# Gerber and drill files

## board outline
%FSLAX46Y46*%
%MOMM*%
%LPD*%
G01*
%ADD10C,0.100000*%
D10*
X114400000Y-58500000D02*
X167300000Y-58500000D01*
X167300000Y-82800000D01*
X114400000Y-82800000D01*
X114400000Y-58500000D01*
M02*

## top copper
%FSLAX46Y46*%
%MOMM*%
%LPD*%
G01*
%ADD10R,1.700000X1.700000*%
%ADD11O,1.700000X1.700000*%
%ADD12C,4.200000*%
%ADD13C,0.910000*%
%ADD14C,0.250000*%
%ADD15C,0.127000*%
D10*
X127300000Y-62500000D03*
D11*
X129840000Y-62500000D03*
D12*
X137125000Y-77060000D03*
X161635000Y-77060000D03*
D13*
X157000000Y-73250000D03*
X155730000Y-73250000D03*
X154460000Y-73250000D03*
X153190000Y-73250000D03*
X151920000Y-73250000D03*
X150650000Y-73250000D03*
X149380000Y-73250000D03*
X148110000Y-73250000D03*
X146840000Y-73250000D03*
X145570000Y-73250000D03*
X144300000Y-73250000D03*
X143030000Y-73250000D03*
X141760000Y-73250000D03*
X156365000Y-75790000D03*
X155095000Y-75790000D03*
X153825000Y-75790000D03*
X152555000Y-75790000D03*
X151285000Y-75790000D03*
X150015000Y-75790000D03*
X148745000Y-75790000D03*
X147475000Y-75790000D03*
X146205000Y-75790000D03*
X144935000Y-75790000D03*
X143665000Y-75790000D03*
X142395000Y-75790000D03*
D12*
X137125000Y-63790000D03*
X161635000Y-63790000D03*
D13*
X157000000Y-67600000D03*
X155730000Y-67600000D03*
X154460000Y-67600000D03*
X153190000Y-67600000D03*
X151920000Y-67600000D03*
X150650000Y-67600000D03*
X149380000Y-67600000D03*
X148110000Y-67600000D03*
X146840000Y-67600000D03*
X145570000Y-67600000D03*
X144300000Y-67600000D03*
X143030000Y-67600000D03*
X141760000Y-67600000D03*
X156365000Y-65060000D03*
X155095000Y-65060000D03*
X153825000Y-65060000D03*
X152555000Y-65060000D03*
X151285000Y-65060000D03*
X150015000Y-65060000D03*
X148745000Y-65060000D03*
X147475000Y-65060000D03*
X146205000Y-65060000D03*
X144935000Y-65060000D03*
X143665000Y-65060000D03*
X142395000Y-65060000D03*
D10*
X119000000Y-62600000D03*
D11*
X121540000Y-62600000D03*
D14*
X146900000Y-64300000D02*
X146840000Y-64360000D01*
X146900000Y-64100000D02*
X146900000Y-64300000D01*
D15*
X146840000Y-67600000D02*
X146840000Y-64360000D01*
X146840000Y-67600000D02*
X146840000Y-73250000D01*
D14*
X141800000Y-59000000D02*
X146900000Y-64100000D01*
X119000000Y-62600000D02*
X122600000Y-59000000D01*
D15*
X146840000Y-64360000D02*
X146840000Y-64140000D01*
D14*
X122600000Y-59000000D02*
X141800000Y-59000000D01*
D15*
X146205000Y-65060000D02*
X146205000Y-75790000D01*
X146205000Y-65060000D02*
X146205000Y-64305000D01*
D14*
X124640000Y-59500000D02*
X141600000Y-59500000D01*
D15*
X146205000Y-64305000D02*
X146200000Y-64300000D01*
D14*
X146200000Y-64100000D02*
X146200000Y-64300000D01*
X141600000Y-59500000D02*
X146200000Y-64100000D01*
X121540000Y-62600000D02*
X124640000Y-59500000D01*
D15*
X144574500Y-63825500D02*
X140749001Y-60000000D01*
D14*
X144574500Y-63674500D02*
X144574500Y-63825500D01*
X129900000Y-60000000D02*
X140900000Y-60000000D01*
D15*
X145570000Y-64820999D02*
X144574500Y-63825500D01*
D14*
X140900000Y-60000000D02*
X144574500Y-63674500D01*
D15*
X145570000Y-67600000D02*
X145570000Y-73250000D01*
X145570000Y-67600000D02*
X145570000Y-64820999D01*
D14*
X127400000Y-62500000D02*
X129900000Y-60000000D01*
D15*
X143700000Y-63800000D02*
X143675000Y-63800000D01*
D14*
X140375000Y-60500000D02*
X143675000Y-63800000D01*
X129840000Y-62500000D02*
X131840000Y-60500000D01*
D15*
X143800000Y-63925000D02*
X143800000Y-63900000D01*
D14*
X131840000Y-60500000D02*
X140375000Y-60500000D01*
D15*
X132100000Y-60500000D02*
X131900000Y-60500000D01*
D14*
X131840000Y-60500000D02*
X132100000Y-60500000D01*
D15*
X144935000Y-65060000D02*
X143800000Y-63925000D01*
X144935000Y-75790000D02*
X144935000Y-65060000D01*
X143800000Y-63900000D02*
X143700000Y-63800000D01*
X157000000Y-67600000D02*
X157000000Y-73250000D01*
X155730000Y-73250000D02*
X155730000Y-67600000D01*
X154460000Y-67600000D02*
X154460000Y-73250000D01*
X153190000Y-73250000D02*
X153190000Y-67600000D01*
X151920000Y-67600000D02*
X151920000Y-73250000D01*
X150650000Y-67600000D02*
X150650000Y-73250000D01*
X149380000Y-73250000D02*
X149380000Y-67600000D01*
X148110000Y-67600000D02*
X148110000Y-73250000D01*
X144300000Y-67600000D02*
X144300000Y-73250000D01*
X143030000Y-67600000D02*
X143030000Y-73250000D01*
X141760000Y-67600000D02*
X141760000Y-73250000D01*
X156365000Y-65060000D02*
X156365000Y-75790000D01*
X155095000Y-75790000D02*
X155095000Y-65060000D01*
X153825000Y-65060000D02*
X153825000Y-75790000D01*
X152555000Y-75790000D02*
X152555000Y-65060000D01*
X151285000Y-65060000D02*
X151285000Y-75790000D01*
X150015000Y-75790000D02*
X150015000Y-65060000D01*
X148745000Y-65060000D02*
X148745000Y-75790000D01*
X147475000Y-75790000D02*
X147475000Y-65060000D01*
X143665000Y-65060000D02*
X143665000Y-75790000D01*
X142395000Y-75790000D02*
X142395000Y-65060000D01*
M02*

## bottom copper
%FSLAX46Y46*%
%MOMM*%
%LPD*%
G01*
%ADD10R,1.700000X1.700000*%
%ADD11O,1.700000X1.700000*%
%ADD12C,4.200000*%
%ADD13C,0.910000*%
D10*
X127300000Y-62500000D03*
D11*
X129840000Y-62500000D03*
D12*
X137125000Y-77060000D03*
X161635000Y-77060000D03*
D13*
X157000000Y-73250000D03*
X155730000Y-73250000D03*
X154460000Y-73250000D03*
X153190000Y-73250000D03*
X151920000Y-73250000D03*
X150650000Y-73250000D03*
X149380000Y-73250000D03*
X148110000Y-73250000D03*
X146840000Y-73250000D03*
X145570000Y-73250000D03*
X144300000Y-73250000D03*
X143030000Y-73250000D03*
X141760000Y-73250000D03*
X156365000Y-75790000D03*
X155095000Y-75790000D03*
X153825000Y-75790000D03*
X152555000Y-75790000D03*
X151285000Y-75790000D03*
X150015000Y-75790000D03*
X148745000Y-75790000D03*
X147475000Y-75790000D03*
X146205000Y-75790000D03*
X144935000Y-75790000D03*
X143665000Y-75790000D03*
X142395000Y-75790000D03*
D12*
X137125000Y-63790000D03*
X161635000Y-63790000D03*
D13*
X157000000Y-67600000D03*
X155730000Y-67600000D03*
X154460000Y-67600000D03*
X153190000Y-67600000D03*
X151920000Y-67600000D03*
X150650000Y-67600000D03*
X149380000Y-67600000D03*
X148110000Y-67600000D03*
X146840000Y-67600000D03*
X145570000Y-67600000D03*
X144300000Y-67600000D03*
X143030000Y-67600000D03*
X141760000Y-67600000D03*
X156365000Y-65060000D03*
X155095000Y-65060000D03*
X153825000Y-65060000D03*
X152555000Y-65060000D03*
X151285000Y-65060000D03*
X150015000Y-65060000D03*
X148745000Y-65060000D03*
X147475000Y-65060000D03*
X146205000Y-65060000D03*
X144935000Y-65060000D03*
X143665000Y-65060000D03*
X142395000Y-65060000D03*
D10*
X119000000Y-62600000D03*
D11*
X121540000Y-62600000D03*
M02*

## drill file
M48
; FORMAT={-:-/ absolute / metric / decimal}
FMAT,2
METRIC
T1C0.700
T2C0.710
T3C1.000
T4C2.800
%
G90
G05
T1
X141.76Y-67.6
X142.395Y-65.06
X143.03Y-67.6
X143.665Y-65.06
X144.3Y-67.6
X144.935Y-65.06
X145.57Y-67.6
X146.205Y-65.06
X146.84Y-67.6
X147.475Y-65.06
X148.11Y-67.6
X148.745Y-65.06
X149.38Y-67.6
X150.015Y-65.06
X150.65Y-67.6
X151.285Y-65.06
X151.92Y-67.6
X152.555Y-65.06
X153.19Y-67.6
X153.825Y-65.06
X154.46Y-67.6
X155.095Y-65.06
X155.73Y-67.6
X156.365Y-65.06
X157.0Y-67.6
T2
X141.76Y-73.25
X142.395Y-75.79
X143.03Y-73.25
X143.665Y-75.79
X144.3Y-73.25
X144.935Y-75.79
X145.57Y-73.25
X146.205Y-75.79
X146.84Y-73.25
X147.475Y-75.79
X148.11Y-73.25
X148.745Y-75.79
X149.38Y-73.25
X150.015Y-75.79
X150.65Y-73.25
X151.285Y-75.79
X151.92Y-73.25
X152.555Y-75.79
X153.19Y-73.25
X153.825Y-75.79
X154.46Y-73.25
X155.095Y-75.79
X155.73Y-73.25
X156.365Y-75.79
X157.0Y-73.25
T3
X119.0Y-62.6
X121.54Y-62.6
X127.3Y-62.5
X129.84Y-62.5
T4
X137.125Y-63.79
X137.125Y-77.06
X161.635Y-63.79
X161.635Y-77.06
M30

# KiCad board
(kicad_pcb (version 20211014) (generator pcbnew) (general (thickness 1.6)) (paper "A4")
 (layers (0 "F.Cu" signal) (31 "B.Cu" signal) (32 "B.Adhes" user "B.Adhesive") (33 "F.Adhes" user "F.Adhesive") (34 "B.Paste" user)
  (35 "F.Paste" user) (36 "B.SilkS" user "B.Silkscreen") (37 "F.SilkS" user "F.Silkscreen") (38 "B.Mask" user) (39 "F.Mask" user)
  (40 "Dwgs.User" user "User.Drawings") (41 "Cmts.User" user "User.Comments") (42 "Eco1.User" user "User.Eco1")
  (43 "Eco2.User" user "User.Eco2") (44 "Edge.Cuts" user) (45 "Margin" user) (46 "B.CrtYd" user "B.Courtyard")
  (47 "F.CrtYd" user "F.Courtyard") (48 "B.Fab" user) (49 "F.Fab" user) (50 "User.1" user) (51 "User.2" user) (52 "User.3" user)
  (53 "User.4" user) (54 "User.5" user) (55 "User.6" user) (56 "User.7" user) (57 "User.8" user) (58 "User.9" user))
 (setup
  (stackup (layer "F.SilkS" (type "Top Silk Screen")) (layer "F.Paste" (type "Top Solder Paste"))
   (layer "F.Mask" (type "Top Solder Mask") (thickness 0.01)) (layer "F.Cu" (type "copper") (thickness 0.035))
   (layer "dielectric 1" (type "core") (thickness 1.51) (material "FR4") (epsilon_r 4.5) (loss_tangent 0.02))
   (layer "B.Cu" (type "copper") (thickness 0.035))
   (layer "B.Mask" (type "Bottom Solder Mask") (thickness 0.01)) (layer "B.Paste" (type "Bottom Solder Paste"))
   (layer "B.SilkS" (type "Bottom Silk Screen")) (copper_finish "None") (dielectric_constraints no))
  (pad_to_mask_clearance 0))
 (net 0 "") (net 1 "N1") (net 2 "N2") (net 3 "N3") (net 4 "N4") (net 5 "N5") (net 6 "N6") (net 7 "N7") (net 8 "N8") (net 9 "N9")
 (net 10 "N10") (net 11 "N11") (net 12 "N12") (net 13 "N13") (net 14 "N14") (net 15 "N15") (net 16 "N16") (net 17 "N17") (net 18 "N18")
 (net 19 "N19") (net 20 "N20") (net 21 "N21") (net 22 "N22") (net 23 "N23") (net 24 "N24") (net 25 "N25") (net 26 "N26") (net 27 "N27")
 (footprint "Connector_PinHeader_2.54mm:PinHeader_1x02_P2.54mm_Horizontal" (layer "F.Cu") (at 127.3 62.5 90)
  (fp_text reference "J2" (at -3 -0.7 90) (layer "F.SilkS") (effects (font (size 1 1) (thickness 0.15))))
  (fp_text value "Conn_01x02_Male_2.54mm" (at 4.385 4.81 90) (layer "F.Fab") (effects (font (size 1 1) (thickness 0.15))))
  (pad "1" thru_hole rect (at 0 0 90) (size 1.7 1.7) (drill 1) (layers *.Cu *.Mask) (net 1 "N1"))
  (pad "2" thru_hole oval (at 0 2.54 90) (size 1.7 1.7) (drill 1) (layers *.Cu *.Mask) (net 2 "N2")))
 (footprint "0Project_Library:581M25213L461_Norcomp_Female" (layer "F.Cu") (at 157 73.25)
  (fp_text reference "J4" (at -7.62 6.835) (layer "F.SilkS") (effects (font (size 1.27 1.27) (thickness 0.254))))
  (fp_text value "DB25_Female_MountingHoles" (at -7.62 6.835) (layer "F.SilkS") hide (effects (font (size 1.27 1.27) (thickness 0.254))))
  (pad "0" thru_hole circle (at -19.875 3.81) (size 4.2 4.2) (drill 2.8) (layers *.Cu *.Mask) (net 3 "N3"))
  (pad "0" thru_hole circle (at 4.635 3.81) (size 4.2 4.2) (drill 2.8) (layers *.Cu *.Mask) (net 3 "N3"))
  (pad "1" thru_hole circle (at 0 0) (size 0.91 0.91) (drill 0.71) (layers *.Cu *.Mask) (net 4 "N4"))
  (pad "2" thru_hole circle (at -1.27 0) (size 0.91 0.91) (drill 0.71) (layers *.Cu *.Mask) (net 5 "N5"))
  (pad "3" thru_hole circle (at -2.54 0) (size 0.91 0.91) (drill 0.71) (layers *.Cu *.Mask) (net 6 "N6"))
  (pad "4" thru_hole circle (at -3.81 0) (size 0.91 0.91) (drill 0.71) (layers *.Cu *.Mask) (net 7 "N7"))
  (pad "5" thru_hole circle (at -5.08 0) (size 0.91 0.91) (drill 0.71) (layers *.Cu *.Mask) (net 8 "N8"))
  (pad "6" thru_hole circle (at -6.35 0) (size 0.91 0.91) (drill 0.71) (layers *.Cu *.Mask) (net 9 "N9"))
  (pad "7" thru_hole circle (at -7.62 0) (size 0.91 0.91) (drill 0.71) (layers *.Cu *.Mask) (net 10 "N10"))
  (pad "8" thru_hole circle (at -8.89 0) (size 0.91 0.91) (drill 0.71) (layers *.Cu *.Mask) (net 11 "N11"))
  (pad "9" thru_hole circle (at -10.16 0) (size 0.91 0.91) (drill 0.71) (layers *.Cu *.Mask) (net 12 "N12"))
  (pad "10" thru_hole circle (at -11.43 0) (size 0.91 0.91) (drill 0.71) (layers *.Cu *.Mask) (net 1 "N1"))
  (pad "11" thru_hole circle (at -12.7 0) (size 0.91 0.91) (drill 0.71) (layers *.Cu *.Mask) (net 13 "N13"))
  (pad "12" thru_hole circle (at -13.97 0) (size 0.91 0.91) (drill 0.71) (layers *.Cu *.Mask) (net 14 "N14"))
  (pad "13" thru_hole circle (at -15.24 0) (size 0.91 0.91) (drill 0.71) (layers *.Cu *.Mask) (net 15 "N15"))
  (pad "14" thru_hole circle (at -0.635 2.54) (size 0.91 0.91) (drill 0.71) (layers *.Cu *.Mask) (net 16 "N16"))
  (pad "15" thru_hole circle (at -1.905 2.54) (size 0.91 0.91) (drill 0.71) (layers *.Cu *.Mask) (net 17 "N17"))
  (pad "16" thru_hole circle (at -3.175 2.54) (size 0.91 0.91) (drill 0.71) (layers *.Cu *.Mask) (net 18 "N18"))
  (pad "17" thru_hole circle (at -4.445 2.54) (size 0.91 0.91) (drill 0.71) (layers *.Cu *.Mask) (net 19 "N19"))
  (pad "18" thru_hole circle (at -5.715 2.54) (size 0.91 0.91) (drill 0.71) (layers *.Cu *.Mask) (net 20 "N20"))
  (pad "19" thru_hole circle (at -6.985 2.54) (size 0.91 0.91) (drill 0.71) (layers *.Cu *.Mask) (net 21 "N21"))
  (pad "20" thru_hole circle (at -8.255 2.54) (size 0.91 0.91) (drill 0.71) (layers *.Cu *.Mask) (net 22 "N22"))
  (pad "21" thru_hole circle (at -9.525 2.54) (size 0.91 0.91) (drill 0.71) (layers *.Cu *.Mask) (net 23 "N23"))
  (pad "22" thru_hole circle (at -10.795 2.54) (size 0.91 0.91) (drill 0.71) (layers *.Cu *.Mask) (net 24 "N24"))
  (pad "23" thru_hole circle (at -12.065 2.54) (size 0.91 0.91) (drill 0.71) (layers *.Cu *.Mask) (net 2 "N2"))
  (pad "24" thru_hole circle (at -13.335 2.54) (size 0.91 0.91) (drill 0.71) (layers *.Cu *.Mask) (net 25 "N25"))
  (pad "25" thru_hole circle (at -14.605 2.54) (size 0.91 0.91) (drill 0.71) (layers *.Cu *.Mask) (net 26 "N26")))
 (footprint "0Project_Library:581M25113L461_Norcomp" (layer "F.Cu") (at 157 67.6 180)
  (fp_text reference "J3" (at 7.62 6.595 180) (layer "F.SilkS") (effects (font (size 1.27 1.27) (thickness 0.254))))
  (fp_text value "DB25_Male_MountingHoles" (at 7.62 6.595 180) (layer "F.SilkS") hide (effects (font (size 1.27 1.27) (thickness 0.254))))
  (pad "0" thru_hole circle (at 19.875 3.81 180) (size 4.2 4.2) (drill 2.8) (layers *.Cu *.Mask) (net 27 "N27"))
  (pad "0" thru_hole circle (at -4.635 3.81 180) (size 4.2 4.2) (drill 2.8) (layers *.Cu *.Mask) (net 27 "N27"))
  (pad "1" thru_hole circle (at 0 0 180) (size 0.91 0.91) (drill 0.7) (layers *.Cu *.Mask) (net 4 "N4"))
  (pad "2" thru_hole circle (at 1.27 0 180) (size 0.91 0.91) (drill 0.7) (layers *.Cu *.Mask) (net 5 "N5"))
  (pad "3" thru_hole circle (at 2.54 0 180) (size 0.91 0.91) (drill 0.7) (layers *.Cu *.Mask) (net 6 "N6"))
  (pad "4" thru_hole circle (at 3.81 0 180) (size 0.91 0.91) (drill 0.7) (layers *.Cu *.Mask) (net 7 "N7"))
  (pad "5" thru_hole circle (at 5.08 0 180) (size 0.91 0.91) (drill 0.7) (layers *.Cu *.Mask) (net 8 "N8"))
  (pad "6" thru_hole circle (at 6.35 0 180) (size 0.91 0.91) (drill 0.7) (layers *.Cu *.Mask) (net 9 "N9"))
  (pad "7" thru_hole circle (at 7.62 0 180) (size 0.91 0.91) (drill 0.7) (layers *.Cu *.Mask) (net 10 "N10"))
  (pad "8" thru_hole circle (at 8.89 0 180) (size 0.91 0.91) (drill 0.7) (layers *.Cu *.Mask) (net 11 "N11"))
  (pad "9" thru_hole circle (at 10.16 0 180) (size 0.91 0.91) (drill 0.7) (layers *.Cu *.Mask) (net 12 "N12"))
  (pad "10" thru_hole circle (at 11.43 0 180) (size 0.91 0.91) (drill 0.7) (layers *.Cu *.Mask) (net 1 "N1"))
  (pad "11" thru_hole circle (at 12.7 0 180) (size 0.91 0.91) (drill 0.7) (layers *.Cu *.Mask) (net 13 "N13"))
  (pad "12" thru_hole circle (at 13.97 0 180) (size 0.91 0.91) (drill 0.7) (layers *.Cu *.Mask) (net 14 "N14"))
  (pad "13" thru_hole circle (at 15.24 0 180) (size 0.91 0.91) (drill 0.7) (layers *.Cu *.Mask) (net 15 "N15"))
  (pad "14" thru_hole circle (at 0.635 2.54 180) (size 0.91 0.91) (drill 0.7) (layers *.Cu *.Mask) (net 16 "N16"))
  (pad "15" thru_hole circle (at 1.905 2.54 180) (size 0.91 0.91) (drill 0.7) (layers *.Cu *.Mask) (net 17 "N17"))
  (pad "16" thru_hole circle (at 3.175 2.54 180) (size 0.91 0.91) (drill 0.7) (layers *.Cu *.Mask) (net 18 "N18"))
  (pad "17" thru_hole circle (at 4.445 2.54 180) (size 0.91 0.91) (drill 0.7) (layers *.Cu *.Mask) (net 19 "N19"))
  (pad "18" thru_hole circle (at 5.715 2.54 180) (size 0.91 0.91) (drill 0.7) (layers *.Cu *.Mask) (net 20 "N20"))
  (pad "19" thru_hole circle (at 6.985 2.54 180) (size 0.91 0.91) (drill 0.7) (layers *.Cu *.Mask) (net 21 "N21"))
  (pad "20" thru_hole circle (at 8.255 2.54 180) (size 0.91 0.91) (drill 0.7) (layers *.Cu *.Mask) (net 22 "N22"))
  (pad "21" thru_hole circle (at 9.525 2.54 180) (size 0.91 0.91) (drill 0.7) (layers *.Cu *.Mask) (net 23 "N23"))
  (pad "22" thru_hole circle (at 10.795 2.54 180) (size 0.91 0.91) (drill 0.7) (layers *.Cu *.Mask) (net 24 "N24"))
  (pad "23" thru_hole circle (at 12.065 2.54 180) (size 0.91 0.91) (drill 0.7) (layers *.Cu *.Mask) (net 2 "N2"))
  (pad "24" thru_hole circle (at 13.335 2.54 180) (size 0.91 0.91) (drill 0.7) (layers *.Cu *.Mask) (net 25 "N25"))
  (pad "25" thru_hole circle (at 14.605 2.54 180) (size 0.91 0.91) (drill 0.7) (layers *.Cu *.Mask) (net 26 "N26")))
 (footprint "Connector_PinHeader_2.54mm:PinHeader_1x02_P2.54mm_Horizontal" (layer "F.Cu") (at 119 62.6 90)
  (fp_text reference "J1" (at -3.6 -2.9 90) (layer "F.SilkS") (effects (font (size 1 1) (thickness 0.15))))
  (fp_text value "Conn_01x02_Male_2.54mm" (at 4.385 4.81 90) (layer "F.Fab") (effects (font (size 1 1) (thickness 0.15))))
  (pad "1" thru_hole rect (at 0 0 90) (size 1.7 1.7) (drill 1) (layers *.Cu *.Mask) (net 12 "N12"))
  (pad "2" thru_hole oval (at 0 2.54 90) (size 1.7 1.7) (drill 1) (layers *.Cu *.Mask) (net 24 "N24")))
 (gr_rect (start 114.4 58.5) (end 167.3 82.8) (layer "Edge.Cuts") (width 0.1) (fill none))
 (segment (start 146.9 64.3) (end 146.84 64.36) (width 0.25) (layer "F.Cu") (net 12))
 (segment (start 146.9 64.1) (end 146.9 64.3) (width 0.25) (layer "F.Cu") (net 12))
 (segment (start 146.84 67.6) (end 146.84 64.36) (width 0.127) (layer "F.Cu") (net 12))
 (segment (start 146.84 67.6) (end 146.84 73.25) (width 0.127) (layer "F.Cu") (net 12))
 (segment (start 141.8 59) (end 146.9 64.1) (width 0.25) (layer "F.Cu") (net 12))
 (segment (start 119 62.6) (end 122.6 59) (width 0.25) (layer "F.Cu") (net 12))
 (segment (start 146.84 64.36) (end 146.84 64.14) (width 0.127) (layer "F.Cu") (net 12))
 (segment (start 122.6 59) (end 141.8 59) (width 0.25) (layer "F.Cu") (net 12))
 (segment (start 146.205 65.06) (end 146.205 75.79) (width 0.127) (layer "F.Cu") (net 24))
 (segment (start 146.205 65.06) (end 146.205 64.305) (width 0.127) (layer "F.Cu") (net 24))
 (segment (start 124.64 59.5) (end 141.6 59.5) (width 0.25) (layer "F.Cu") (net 24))
 (segment (start 146.205 64.305) (end 146.2 64.3) (width 0.127) (layer "F.Cu") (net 24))
 (segment (start 146.2 64.1) (end 146.2 64.3) (width 0.25) (layer "F.Cu") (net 24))
 (segment (start 141.6 59.5) (end 146.2 64.1) (width 0.25) (layer "F.Cu") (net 24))
 (segment (start 121.54 62.6) (end 124.64 59.5) (width 0.25) (layer "F.Cu") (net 24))
 (segment (start 144.5745 63.8255) (end 140.749001 60) (width 0.127) (layer "F.Cu") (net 1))
 (segment (start 144.5745 63.6745) (end 144.5745 63.8255) (width 0.25) (layer "F.Cu") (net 1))
 (segment (start 129.9 60) (end 140.9 60) (width 0.25) (layer "F.Cu") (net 1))
 (segment (start 145.57 64.820999) (end 144.5745 63.8255) (width 0.127) (layer "F.Cu") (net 1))
 (segment (start 140.9 60) (end 144.5745 63.6745) (width 0.25) (layer "F.Cu") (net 1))
 (segment (start 145.57 67.6) (end 145.57 73.25) (width 0.127) (layer "F.Cu") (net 1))
 (segment (start 145.57 67.6) (end 145.57 64.820999) (width 0.127) (layer "F.Cu") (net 1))
 (segment (start 127.4 62.5) (end 129.9 60) (width 0.25) (layer "F.Cu") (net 1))
 (segment (start 143.7 63.8) (end 143.675 63.8) (width 0.127) (layer "F.Cu") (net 2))
 (segment (start 140.375 60.5) (end 143.675 63.8) (width 0.25) (layer "F.Cu") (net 2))
 (segment (start 129.84 62.5) (end 131.84 60.5) (width 0.25) (layer "F.Cu") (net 2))
 (segment (start 143.8 63.925) (end 143.8 63.9) (width 0.127) (layer "F.Cu") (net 2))
 (segment (start 131.84 60.5) (end 140.375 60.5) (width 0.25) (layer "F.Cu") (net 2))
 (segment (start 132.1 60.5) (end 131.9 60.5) (width 0.127) (layer "F.Cu") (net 2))
 (segment (start 131.84 60.5) (end 132.1 60.5) (width 0.25) (layer "F.Cu") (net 2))
 (segment (start 144.935 65.06) (end 143.8 63.925) (width 0.127) (layer "F.Cu") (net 2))
 (segment (start 144.935 75.79) (end 144.935 65.06) (width 0.127) (layer "F.Cu") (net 2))
 (segment (start 143.8 63.9) (end 143.7 63.8) (width 0.127) (layer "F.Cu") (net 2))
 (segment (start 157 67.6) (end 157 73.25) (width 0.127) (layer "F.Cu") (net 4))
 (segment (start 155.73 73.25) (end 155.73 67.6) (width 0.127) (layer "F.Cu") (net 5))
 (segment (start 154.46 67.6) (end 154.46 73.25) (width 0.127) (layer "F.Cu") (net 6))
 (segment (start 153.19 73.25) (end 153.19 67.6) (width 0.127) (layer "F.Cu") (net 7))
 (segment (start 151.92 67.6) (end 151.92 73.25) (width 0.127) (layer "F.Cu") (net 8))
 (segment (start 150.65 67.6) (end 150.65 73.25) (width 0.127) (layer "F.Cu") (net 9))
 (segment (start 149.38 73.25) (end 149.38 67.6) (width 0.127) (layer "F.Cu") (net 10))
 (segment (start 148.11 67.6) (end 148.11 73.25) (width 0.127) (layer "F.Cu") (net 11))
 (segment (start 144.3 67.6) (end 144.3 73.25) (width 0.127) (layer "F.Cu") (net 13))
 (segment (start 143.03 67.6) (end 143.03 73.25) (width 0.127) (layer "F.Cu") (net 14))
 (segment (start 141.76 67.6) (end 141.76 73.25) (width 0.127) (layer "F.Cu") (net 15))
 (segment (start 156.365 65.06) (end 156.365 75.79) (width 0.127) (layer "F.Cu") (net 16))
 (segment (start 155.095 75.79) (end 155.095 65.06) (width 0.127) (layer "F.Cu") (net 17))
 (segment (start 153.825 65.06) (end 153.825 75.79) (width 0.127) (layer "F.Cu") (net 18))
 (segment (start 152.555 75.79) (end 152.555 65.06) (width 0.127) (layer "F.Cu") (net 19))
 (segment (start 151.285 65.06) (end 151.285 75.79) (width 0.127) (layer "F.Cu") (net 20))
 (segment (start 150.015 75.79) (end 150.015 65.06) (width 0.127) (layer "F.Cu") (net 21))
 (segment (start 148.745 65.06) (end 148.745 75.79) (width 0.127) (layer "F.Cu") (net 22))
 (segment (start 147.475 75.79) (end 147.475 65.06) (width 0.127) (layer "F.Cu") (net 23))
 (segment (start 143.665 65.06) (end 143.665 75.79) (width 0.127) (layer "F.Cu") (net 25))
 (segment (start 142.395 75.79) (end 142.395 65.06) (width 0.127) (layer "F.Cu") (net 26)))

